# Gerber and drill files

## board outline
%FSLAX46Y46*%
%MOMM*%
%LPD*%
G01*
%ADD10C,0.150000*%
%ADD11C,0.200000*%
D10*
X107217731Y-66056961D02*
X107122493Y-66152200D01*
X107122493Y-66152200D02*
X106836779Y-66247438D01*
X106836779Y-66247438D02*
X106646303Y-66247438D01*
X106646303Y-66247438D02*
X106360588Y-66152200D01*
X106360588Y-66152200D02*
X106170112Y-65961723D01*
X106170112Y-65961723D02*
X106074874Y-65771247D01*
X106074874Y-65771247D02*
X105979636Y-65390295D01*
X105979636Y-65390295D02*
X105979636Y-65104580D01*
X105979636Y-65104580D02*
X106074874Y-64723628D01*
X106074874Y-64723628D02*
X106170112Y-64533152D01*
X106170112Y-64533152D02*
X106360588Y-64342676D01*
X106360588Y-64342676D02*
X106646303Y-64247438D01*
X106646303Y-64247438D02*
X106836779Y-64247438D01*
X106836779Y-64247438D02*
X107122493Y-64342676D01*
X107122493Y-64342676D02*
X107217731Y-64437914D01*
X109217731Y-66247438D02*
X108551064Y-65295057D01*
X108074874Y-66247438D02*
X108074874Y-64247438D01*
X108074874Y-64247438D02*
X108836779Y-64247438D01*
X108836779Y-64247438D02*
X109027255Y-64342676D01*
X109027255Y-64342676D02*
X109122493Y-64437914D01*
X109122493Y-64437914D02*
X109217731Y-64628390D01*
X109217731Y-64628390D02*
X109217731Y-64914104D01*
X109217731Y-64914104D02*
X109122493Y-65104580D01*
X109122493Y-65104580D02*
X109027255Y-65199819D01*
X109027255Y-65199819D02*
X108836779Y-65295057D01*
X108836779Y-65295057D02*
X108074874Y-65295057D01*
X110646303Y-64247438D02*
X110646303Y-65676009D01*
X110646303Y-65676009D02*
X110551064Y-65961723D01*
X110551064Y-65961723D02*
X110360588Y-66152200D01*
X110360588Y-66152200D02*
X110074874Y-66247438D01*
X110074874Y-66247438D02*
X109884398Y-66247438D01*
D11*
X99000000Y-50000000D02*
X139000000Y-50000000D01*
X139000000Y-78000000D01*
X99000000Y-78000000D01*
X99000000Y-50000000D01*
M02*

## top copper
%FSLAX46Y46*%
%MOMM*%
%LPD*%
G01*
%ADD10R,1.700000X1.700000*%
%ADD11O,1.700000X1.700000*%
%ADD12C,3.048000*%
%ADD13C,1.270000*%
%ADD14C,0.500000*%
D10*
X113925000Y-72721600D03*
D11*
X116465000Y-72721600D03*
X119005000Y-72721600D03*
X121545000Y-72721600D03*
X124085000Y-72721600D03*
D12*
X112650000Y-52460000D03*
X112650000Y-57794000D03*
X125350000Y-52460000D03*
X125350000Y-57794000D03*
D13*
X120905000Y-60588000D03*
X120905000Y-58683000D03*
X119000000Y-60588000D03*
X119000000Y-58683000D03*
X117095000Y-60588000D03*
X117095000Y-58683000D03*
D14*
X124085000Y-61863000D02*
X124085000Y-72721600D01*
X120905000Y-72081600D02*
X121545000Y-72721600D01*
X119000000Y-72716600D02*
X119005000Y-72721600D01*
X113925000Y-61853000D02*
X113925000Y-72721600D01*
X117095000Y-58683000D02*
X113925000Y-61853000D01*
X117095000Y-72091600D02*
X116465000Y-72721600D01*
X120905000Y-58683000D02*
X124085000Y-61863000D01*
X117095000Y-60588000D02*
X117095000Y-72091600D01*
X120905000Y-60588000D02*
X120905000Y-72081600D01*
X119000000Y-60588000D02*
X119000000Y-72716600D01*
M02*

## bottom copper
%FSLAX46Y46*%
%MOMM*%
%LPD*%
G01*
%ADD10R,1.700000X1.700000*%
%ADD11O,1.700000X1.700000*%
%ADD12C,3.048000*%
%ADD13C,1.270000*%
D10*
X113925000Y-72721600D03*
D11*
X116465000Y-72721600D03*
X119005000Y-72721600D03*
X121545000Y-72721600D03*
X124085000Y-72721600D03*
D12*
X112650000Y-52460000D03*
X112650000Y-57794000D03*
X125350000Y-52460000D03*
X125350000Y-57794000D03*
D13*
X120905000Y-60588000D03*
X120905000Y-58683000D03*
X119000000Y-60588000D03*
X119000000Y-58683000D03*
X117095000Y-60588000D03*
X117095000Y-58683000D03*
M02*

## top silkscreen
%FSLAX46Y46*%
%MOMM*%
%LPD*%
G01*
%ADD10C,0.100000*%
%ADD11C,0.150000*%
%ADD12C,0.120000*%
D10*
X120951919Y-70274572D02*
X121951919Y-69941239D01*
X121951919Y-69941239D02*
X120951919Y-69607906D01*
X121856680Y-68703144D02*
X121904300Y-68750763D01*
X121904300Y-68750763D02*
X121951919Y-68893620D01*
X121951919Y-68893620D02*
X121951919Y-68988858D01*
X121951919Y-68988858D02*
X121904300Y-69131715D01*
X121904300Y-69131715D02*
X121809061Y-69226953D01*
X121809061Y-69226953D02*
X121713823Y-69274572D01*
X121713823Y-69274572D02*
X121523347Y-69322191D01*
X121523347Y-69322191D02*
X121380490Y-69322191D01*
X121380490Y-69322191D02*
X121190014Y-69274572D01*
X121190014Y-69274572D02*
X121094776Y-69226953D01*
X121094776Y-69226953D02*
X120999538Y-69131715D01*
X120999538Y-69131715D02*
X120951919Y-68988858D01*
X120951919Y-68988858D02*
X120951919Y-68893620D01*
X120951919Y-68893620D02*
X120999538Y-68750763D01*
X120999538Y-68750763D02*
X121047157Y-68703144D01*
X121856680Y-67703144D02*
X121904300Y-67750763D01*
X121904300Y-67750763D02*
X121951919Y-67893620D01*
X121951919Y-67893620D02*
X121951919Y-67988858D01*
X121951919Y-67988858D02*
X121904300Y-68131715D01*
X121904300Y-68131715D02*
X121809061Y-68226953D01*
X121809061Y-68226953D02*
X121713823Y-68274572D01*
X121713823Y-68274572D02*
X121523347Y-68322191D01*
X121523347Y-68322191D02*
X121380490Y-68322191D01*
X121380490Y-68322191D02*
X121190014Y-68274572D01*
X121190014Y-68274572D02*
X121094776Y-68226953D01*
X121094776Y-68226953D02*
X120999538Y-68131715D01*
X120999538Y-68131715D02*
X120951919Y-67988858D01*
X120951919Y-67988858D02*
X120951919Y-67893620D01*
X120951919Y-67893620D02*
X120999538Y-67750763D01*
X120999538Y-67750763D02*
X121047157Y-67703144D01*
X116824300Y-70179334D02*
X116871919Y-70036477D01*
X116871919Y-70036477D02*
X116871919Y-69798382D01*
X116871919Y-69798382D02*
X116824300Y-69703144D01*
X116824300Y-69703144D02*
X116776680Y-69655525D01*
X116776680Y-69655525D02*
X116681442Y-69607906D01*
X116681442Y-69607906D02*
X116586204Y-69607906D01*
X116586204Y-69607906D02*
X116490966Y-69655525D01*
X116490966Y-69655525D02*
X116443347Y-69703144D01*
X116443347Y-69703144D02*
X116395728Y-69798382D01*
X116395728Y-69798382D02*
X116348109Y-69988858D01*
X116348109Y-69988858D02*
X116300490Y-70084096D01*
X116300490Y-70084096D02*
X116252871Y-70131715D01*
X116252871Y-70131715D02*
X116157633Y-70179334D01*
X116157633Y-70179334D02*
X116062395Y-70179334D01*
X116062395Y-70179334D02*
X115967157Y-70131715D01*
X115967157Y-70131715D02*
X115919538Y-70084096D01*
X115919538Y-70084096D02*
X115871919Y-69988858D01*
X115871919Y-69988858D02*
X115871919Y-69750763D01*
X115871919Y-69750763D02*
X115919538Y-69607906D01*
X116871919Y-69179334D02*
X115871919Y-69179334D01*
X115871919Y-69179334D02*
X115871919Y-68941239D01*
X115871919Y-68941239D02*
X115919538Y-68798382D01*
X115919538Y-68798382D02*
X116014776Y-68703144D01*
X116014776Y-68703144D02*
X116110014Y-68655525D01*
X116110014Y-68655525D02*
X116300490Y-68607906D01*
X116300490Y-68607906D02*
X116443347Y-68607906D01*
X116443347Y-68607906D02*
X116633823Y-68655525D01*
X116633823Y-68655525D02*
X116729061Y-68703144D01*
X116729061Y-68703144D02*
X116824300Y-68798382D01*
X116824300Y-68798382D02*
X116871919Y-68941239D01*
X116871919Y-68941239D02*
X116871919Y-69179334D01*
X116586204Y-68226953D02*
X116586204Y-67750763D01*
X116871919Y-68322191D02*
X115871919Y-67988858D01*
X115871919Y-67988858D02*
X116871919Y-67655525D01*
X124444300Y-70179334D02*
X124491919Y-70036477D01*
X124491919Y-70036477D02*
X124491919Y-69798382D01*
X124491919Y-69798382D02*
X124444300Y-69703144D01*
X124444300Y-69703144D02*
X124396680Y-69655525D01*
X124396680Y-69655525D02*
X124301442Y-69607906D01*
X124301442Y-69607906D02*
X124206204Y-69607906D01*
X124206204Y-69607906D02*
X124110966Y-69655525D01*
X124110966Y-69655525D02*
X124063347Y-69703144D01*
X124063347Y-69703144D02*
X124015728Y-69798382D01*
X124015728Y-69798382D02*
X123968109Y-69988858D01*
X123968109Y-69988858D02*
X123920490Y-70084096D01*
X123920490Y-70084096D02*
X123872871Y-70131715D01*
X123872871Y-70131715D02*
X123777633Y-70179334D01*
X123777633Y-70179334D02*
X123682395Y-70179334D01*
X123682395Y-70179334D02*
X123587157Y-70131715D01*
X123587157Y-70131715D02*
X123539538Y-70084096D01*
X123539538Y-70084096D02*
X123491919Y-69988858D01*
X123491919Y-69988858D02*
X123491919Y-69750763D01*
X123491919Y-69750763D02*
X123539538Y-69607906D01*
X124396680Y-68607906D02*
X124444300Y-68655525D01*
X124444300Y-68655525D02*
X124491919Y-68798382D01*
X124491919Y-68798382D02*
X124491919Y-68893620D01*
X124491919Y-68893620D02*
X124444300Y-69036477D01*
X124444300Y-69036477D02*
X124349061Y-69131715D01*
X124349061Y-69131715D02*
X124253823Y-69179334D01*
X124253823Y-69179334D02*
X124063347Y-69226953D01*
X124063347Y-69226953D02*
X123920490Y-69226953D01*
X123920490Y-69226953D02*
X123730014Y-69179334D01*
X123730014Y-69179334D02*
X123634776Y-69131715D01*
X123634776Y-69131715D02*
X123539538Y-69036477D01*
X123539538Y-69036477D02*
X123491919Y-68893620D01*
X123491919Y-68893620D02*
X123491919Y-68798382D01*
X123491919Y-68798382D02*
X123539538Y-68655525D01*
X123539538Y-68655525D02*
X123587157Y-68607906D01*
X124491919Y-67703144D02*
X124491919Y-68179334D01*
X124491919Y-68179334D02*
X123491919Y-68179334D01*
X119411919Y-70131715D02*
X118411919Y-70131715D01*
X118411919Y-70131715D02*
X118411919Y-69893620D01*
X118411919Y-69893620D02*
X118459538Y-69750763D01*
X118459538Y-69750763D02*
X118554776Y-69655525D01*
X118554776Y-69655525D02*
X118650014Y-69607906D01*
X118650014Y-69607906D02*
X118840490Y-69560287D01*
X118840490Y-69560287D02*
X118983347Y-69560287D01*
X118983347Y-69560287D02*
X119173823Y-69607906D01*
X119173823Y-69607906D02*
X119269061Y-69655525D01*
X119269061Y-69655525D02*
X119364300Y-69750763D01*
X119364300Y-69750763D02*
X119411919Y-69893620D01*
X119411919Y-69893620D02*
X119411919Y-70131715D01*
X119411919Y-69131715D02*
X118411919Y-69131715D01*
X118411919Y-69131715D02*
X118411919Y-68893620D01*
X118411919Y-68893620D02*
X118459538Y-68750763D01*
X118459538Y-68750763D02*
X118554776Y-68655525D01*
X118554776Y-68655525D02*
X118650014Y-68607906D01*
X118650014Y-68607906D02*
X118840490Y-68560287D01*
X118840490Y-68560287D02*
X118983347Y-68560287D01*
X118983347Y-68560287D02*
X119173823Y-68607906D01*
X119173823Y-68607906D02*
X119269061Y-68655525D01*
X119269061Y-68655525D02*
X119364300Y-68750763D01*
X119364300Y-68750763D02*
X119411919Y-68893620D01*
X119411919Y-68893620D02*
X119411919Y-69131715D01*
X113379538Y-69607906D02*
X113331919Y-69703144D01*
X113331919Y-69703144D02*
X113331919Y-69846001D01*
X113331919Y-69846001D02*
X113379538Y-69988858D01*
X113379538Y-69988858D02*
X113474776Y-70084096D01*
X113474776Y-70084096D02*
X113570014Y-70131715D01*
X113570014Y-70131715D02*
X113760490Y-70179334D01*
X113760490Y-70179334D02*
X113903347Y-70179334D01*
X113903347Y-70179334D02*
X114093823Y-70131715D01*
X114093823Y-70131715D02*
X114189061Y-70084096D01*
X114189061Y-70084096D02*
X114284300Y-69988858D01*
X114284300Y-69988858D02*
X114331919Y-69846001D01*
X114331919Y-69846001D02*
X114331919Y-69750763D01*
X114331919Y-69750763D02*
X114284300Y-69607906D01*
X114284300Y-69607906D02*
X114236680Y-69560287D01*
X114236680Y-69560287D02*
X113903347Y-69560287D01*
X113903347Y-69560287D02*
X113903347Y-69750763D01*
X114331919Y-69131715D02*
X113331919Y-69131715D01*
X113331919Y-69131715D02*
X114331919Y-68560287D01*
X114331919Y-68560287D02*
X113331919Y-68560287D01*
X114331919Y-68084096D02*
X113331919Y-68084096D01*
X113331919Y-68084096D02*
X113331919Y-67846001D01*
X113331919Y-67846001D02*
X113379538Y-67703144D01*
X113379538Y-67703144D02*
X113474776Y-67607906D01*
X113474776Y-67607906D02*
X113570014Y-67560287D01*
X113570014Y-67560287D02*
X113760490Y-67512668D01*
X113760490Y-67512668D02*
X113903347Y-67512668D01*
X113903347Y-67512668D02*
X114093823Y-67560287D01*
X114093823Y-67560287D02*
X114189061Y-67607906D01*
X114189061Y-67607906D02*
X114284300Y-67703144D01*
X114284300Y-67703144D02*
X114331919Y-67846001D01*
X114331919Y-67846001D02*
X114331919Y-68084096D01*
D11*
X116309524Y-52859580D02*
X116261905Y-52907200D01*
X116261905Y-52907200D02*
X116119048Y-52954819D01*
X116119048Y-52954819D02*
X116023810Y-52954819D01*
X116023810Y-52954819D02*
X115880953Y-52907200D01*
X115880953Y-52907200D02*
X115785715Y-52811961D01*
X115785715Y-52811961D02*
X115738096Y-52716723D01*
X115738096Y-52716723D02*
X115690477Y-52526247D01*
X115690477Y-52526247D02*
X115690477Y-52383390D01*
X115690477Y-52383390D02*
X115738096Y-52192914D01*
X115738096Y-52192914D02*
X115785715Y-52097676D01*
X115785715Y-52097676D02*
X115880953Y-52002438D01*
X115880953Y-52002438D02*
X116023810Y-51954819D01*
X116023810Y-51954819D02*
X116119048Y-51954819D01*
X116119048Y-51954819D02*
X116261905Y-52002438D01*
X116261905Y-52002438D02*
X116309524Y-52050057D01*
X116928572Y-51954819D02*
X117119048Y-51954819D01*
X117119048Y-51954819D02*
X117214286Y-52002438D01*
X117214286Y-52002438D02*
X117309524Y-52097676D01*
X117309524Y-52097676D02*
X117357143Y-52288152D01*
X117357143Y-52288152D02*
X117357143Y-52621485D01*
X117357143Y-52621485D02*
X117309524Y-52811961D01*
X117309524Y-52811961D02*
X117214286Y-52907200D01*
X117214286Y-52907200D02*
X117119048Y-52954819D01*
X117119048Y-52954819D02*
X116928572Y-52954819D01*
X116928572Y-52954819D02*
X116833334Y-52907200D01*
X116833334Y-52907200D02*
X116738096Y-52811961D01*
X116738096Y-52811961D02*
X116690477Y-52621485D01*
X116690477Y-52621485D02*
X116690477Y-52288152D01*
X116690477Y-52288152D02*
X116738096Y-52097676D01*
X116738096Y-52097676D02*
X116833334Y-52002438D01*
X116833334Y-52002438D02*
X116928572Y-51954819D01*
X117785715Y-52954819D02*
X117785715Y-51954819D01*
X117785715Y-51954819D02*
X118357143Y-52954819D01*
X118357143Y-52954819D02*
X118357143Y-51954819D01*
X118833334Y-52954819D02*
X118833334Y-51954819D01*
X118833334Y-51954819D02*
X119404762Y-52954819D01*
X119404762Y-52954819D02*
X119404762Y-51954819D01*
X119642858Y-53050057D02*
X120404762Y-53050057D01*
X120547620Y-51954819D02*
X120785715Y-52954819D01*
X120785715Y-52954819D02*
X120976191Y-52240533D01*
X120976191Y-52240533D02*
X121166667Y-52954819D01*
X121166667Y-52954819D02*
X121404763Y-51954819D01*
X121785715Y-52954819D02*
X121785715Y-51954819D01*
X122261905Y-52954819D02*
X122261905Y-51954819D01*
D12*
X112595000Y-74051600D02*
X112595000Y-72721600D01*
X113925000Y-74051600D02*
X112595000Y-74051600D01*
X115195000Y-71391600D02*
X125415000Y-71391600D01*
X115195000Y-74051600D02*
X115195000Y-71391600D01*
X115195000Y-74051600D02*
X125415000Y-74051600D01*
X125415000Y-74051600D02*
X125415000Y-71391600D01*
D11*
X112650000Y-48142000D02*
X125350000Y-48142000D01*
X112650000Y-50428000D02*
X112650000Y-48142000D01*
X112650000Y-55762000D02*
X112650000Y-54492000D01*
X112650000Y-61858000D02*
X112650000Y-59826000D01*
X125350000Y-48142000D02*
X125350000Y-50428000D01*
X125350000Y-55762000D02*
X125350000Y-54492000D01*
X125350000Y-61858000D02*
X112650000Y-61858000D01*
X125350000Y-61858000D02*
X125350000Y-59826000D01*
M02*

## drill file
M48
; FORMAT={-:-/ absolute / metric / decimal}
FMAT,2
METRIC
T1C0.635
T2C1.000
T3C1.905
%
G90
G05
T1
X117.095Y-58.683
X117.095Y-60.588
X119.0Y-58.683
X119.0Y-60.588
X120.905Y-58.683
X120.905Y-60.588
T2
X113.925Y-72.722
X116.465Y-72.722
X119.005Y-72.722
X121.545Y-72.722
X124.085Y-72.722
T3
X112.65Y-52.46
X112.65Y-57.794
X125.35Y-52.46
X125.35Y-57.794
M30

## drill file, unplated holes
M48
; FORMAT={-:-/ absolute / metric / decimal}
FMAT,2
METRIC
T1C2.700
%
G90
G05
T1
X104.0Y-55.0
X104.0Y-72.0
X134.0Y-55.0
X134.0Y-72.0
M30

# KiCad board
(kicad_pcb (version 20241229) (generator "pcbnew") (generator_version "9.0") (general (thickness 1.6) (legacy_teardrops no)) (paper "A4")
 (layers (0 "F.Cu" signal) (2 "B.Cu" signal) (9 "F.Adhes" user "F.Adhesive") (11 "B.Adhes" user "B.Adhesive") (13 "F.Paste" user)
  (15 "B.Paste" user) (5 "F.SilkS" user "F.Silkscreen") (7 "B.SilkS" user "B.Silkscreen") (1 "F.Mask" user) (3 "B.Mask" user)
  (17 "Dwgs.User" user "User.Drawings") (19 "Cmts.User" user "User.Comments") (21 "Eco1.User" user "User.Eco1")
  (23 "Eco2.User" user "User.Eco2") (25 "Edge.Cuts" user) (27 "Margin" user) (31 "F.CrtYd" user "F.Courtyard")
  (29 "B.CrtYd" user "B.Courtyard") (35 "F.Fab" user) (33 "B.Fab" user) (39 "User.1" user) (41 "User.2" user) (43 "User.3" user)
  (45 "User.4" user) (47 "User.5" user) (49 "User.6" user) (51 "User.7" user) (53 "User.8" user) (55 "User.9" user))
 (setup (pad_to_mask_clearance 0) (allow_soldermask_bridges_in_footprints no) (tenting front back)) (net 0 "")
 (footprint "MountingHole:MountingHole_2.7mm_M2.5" (layer "F.Cu") (at 134 72)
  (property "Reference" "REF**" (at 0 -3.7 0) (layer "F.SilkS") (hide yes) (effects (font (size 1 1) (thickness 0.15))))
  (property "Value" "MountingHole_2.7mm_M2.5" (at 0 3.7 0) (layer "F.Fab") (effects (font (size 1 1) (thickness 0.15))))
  (pad "" np_thru_hole circle (at 0 0) (size 2.7 2.7) (drill 2.7) (layers "*.Cu" "*.Mask")))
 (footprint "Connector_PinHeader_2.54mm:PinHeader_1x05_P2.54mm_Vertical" (layer "F.Cu") (at 113.925 72.7216 90)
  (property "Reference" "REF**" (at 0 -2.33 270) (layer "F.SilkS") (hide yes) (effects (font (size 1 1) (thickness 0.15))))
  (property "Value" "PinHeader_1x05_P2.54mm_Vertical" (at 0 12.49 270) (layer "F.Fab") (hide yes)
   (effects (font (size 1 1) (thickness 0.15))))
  (fp_line (start -1.33 -1.33) (end 0 -1.33) (stroke (width 0.12) (type solid)) (layer "F.SilkS"))
  (fp_line (start -1.33 0) (end -1.33 -1.33) (stroke (width 0.12) (type solid)) (layer "F.SilkS"))
  (fp_line (start 1.33 1.27) (end 1.33 11.49) (stroke (width 0.12) (type solid)) (layer "F.SilkS"))
  (fp_line (start -1.33 1.27) (end 1.33 1.27) (stroke (width 0.12) (type solid)) (layer "F.SilkS"))
  (fp_line (start -1.33 1.27) (end -1.33 11.49) (stroke (width 0.12) (type solid)) (layer "F.SilkS"))
  (fp_line (start -1.33 11.49) (end 1.33 11.49) (stroke (width 0.12) (type solid)) (layer "F.SilkS"))
  (pad "1" thru_hole rect (at 0 0 90) (size 1.7 1.7) (drill 1) (layers "*.Cu" "*.Mask") (remove_unused_layers no))
  (pad "2" thru_hole oval (at 0 2.54 90) (size 1.7 1.7) (drill 1) (layers "*.Cu" "*.Mask") (remove_unused_layers no))
  (pad "3" thru_hole oval (at 0 5.08 90) (size 1.7 1.7) (drill 1) (layers "*.Cu" "*.Mask") (remove_unused_layers no))
  (pad "4" thru_hole oval (at 0 7.62 90) (size 1.7 1.7) (drill 1) (layers "*.Cu" "*.Mask") (remove_unused_layers no))
  (pad "5" thru_hole oval (at 0 10.16 90) (size 1.7 1.7) (drill 1) (layers "*.Cu" "*.Mask") (remove_unused_layers no)))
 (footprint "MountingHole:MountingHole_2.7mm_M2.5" (layer "F.Cu") (at 104 55)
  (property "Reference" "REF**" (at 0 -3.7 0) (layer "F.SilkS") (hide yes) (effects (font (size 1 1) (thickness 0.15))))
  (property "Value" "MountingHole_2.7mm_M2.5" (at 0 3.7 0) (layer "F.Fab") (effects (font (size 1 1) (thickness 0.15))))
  (pad "" np_thru_hole circle (at 0 0) (size 2.7 2.7) (drill 2.7) (layers "*.Cu" "*.Mask")))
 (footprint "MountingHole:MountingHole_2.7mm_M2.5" (layer "F.Cu") (at 104 72)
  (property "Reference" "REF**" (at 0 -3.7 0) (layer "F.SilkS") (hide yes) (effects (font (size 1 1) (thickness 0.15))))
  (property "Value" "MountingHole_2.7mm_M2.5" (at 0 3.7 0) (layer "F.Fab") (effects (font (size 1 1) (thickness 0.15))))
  (pad "" np_thru_hole circle (at 0 0) (size 2.7 2.7) (drill 2.7) (layers "*.Cu" "*.Mask")))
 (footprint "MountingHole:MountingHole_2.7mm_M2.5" (layer "F.Cu") (at 134 55)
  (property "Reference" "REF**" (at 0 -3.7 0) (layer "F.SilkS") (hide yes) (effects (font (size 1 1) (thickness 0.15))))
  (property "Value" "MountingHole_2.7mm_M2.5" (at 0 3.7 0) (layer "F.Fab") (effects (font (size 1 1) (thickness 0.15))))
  (pad "" np_thru_hole circle (at 0 0) (size 2.7 2.7) (drill 2.7) (layers "*.Cu" "*.Mask")))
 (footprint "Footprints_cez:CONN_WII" (layer "F.Cu") (at 119 55)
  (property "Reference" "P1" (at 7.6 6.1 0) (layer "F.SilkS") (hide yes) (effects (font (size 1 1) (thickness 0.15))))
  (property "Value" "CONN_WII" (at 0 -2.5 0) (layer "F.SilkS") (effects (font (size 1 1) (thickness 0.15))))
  (fp_line (start -6.35 -6.858) (end 6.35 -6.858) (stroke (width 0.15) (type solid)) (layer "F.SilkS"))
  (fp_line (start -6.35 -4.572) (end -6.35 -6.858) (stroke (width 0.15) (type solid)) (layer "F.SilkS"))
  (fp_line (start -6.35 0.762) (end -6.35 -0.508) (stroke (width 0.15) (type solid)) (layer "F.SilkS"))
  (fp_line (start -6.35 6.858) (end -6.35 4.826) (stroke (width 0.15) (type solid)) (layer "F.SilkS"))
  (fp_line (start 6.35 -6.858) (end 6.35 -4.572) (stroke (width 0.15) (type solid)) (layer "F.SilkS"))
  (fp_line (start 6.35 0.762) (end 6.35 -0.508) (stroke (width 0.15) (type solid)) (layer "F.SilkS"))
  (fp_line (start 6.35 6.858) (end -6.35 6.858) (stroke (width 0.15) (type solid)) (layer "F.SilkS"))
  (fp_line (start 6.35 6.858) (end 6.35 4.826) (stroke (width 0.15) (type solid)) (layer "F.SilkS"))
  (pad "" thru_hole circle (at -6.35 -2.54) (size 3.048 3.048) (drill 1.905) (layers "*.Cu" "*.Mask") (remove_unused_layers no))
  (pad "" thru_hole circle (at -6.35 2.794) (size 3.048 3.048) (drill 1.905) (layers "*.Cu" "*.Mask") (remove_unused_layers no))
  (pad "" thru_hole circle (at 6.35 -2.54) (size 3.048 3.048) (drill 1.905) (layers "*.Cu" "*.Mask") (remove_unused_layers no))
  (pad "" thru_hole circle (at 6.35 2.794) (size 3.048 3.048) (drill 1.905) (layers "*.Cu" "*.Mask") (remove_unused_layers no))
  (pad "1" thru_hole circle (at 1.905 5.588) (size 1.27 1.27) (drill 0.635) (layers "*.Cu" "*.Mask") (remove_unused_layers no))
  (pad "2" thru_hole circle (at 1.905 3.683) (size 1.27 1.27) (drill 0.635) (layers "*.Cu" "*.Mask") (remove_unused_layers no))
  (pad "3" thru_hole circle (at 0 5.588) (size 1.27 1.27) (drill 0.635) (layers "*.Cu" "*.Mask") (remove_unused_layers no))
  (pad "4" thru_hole circle (at 0 3.683) (size 1.27 1.27) (drill 0.635) (layers "*.Cu" "*.Mask") (remove_unused_layers no))
  (pad "5" thru_hole circle (at -1.905 5.588) (size 1.27 1.27) (drill 0.635) (layers "*.Cu" "*.Mask") (remove_unused_layers no))
  (pad "6" thru_hole circle (at -1.905 3.683) (size 1.27 1.27) (drill 0.635) (layers "*.Cu" "*.Mask") (remove_unused_layers no)))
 (gr_rect (start 99 50) (end 139 78) (stroke (width 0.2) (type solid)) (fill no) (layer "Edge.Cuts"))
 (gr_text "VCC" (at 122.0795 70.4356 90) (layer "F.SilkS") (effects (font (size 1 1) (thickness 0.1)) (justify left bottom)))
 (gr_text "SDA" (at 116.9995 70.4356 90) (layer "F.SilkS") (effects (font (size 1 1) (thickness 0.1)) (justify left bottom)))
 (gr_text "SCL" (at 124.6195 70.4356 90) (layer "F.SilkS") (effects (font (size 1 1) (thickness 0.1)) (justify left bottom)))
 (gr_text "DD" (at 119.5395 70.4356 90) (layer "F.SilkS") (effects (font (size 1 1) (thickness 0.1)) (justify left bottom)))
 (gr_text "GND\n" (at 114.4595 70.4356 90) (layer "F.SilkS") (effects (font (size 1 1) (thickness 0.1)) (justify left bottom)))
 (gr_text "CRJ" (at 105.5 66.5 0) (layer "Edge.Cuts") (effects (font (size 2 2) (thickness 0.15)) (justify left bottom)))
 (segment (start 117.095 60.588) (end 117.095 72.0916) (width 0.5) (layer "F.Cu") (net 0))
 (segment (start 119 72.7166) (end 119.005 72.7216) (width 0.5) (layer "F.Cu") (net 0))
 (segment (start 113.925 61.853) (end 113.925 72.7216) (width 0.5) (layer "F.Cu") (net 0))
 (segment (start 120.905 60.588) (end 120.905 72.0816) (width 0.5) (layer "F.Cu") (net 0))
 (segment (start 120.905 72.0816) (end 121.545 72.7216) (width 0.5) (layer "F.Cu") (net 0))
 (segment (start 120.905 58.683) (end 124.085 61.863) (width 0.5) (layer "F.Cu") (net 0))
 (segment (start 119 60.588) (end 119 72.7166) (width 0.5) (layer "F.Cu") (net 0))
 (segment (start 117.095 72.0916) (end 116.465 72.7216) (width 0.5) (layer "F.Cu") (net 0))
 (segment (start 117.095 58.683) (end 113.925 61.853) (width 0.5) (layer "F.Cu") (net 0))
 (segment (start 124.085 61.863) (end 124.085 72.7216) (width 0.5) (layer "F.Cu") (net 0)))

